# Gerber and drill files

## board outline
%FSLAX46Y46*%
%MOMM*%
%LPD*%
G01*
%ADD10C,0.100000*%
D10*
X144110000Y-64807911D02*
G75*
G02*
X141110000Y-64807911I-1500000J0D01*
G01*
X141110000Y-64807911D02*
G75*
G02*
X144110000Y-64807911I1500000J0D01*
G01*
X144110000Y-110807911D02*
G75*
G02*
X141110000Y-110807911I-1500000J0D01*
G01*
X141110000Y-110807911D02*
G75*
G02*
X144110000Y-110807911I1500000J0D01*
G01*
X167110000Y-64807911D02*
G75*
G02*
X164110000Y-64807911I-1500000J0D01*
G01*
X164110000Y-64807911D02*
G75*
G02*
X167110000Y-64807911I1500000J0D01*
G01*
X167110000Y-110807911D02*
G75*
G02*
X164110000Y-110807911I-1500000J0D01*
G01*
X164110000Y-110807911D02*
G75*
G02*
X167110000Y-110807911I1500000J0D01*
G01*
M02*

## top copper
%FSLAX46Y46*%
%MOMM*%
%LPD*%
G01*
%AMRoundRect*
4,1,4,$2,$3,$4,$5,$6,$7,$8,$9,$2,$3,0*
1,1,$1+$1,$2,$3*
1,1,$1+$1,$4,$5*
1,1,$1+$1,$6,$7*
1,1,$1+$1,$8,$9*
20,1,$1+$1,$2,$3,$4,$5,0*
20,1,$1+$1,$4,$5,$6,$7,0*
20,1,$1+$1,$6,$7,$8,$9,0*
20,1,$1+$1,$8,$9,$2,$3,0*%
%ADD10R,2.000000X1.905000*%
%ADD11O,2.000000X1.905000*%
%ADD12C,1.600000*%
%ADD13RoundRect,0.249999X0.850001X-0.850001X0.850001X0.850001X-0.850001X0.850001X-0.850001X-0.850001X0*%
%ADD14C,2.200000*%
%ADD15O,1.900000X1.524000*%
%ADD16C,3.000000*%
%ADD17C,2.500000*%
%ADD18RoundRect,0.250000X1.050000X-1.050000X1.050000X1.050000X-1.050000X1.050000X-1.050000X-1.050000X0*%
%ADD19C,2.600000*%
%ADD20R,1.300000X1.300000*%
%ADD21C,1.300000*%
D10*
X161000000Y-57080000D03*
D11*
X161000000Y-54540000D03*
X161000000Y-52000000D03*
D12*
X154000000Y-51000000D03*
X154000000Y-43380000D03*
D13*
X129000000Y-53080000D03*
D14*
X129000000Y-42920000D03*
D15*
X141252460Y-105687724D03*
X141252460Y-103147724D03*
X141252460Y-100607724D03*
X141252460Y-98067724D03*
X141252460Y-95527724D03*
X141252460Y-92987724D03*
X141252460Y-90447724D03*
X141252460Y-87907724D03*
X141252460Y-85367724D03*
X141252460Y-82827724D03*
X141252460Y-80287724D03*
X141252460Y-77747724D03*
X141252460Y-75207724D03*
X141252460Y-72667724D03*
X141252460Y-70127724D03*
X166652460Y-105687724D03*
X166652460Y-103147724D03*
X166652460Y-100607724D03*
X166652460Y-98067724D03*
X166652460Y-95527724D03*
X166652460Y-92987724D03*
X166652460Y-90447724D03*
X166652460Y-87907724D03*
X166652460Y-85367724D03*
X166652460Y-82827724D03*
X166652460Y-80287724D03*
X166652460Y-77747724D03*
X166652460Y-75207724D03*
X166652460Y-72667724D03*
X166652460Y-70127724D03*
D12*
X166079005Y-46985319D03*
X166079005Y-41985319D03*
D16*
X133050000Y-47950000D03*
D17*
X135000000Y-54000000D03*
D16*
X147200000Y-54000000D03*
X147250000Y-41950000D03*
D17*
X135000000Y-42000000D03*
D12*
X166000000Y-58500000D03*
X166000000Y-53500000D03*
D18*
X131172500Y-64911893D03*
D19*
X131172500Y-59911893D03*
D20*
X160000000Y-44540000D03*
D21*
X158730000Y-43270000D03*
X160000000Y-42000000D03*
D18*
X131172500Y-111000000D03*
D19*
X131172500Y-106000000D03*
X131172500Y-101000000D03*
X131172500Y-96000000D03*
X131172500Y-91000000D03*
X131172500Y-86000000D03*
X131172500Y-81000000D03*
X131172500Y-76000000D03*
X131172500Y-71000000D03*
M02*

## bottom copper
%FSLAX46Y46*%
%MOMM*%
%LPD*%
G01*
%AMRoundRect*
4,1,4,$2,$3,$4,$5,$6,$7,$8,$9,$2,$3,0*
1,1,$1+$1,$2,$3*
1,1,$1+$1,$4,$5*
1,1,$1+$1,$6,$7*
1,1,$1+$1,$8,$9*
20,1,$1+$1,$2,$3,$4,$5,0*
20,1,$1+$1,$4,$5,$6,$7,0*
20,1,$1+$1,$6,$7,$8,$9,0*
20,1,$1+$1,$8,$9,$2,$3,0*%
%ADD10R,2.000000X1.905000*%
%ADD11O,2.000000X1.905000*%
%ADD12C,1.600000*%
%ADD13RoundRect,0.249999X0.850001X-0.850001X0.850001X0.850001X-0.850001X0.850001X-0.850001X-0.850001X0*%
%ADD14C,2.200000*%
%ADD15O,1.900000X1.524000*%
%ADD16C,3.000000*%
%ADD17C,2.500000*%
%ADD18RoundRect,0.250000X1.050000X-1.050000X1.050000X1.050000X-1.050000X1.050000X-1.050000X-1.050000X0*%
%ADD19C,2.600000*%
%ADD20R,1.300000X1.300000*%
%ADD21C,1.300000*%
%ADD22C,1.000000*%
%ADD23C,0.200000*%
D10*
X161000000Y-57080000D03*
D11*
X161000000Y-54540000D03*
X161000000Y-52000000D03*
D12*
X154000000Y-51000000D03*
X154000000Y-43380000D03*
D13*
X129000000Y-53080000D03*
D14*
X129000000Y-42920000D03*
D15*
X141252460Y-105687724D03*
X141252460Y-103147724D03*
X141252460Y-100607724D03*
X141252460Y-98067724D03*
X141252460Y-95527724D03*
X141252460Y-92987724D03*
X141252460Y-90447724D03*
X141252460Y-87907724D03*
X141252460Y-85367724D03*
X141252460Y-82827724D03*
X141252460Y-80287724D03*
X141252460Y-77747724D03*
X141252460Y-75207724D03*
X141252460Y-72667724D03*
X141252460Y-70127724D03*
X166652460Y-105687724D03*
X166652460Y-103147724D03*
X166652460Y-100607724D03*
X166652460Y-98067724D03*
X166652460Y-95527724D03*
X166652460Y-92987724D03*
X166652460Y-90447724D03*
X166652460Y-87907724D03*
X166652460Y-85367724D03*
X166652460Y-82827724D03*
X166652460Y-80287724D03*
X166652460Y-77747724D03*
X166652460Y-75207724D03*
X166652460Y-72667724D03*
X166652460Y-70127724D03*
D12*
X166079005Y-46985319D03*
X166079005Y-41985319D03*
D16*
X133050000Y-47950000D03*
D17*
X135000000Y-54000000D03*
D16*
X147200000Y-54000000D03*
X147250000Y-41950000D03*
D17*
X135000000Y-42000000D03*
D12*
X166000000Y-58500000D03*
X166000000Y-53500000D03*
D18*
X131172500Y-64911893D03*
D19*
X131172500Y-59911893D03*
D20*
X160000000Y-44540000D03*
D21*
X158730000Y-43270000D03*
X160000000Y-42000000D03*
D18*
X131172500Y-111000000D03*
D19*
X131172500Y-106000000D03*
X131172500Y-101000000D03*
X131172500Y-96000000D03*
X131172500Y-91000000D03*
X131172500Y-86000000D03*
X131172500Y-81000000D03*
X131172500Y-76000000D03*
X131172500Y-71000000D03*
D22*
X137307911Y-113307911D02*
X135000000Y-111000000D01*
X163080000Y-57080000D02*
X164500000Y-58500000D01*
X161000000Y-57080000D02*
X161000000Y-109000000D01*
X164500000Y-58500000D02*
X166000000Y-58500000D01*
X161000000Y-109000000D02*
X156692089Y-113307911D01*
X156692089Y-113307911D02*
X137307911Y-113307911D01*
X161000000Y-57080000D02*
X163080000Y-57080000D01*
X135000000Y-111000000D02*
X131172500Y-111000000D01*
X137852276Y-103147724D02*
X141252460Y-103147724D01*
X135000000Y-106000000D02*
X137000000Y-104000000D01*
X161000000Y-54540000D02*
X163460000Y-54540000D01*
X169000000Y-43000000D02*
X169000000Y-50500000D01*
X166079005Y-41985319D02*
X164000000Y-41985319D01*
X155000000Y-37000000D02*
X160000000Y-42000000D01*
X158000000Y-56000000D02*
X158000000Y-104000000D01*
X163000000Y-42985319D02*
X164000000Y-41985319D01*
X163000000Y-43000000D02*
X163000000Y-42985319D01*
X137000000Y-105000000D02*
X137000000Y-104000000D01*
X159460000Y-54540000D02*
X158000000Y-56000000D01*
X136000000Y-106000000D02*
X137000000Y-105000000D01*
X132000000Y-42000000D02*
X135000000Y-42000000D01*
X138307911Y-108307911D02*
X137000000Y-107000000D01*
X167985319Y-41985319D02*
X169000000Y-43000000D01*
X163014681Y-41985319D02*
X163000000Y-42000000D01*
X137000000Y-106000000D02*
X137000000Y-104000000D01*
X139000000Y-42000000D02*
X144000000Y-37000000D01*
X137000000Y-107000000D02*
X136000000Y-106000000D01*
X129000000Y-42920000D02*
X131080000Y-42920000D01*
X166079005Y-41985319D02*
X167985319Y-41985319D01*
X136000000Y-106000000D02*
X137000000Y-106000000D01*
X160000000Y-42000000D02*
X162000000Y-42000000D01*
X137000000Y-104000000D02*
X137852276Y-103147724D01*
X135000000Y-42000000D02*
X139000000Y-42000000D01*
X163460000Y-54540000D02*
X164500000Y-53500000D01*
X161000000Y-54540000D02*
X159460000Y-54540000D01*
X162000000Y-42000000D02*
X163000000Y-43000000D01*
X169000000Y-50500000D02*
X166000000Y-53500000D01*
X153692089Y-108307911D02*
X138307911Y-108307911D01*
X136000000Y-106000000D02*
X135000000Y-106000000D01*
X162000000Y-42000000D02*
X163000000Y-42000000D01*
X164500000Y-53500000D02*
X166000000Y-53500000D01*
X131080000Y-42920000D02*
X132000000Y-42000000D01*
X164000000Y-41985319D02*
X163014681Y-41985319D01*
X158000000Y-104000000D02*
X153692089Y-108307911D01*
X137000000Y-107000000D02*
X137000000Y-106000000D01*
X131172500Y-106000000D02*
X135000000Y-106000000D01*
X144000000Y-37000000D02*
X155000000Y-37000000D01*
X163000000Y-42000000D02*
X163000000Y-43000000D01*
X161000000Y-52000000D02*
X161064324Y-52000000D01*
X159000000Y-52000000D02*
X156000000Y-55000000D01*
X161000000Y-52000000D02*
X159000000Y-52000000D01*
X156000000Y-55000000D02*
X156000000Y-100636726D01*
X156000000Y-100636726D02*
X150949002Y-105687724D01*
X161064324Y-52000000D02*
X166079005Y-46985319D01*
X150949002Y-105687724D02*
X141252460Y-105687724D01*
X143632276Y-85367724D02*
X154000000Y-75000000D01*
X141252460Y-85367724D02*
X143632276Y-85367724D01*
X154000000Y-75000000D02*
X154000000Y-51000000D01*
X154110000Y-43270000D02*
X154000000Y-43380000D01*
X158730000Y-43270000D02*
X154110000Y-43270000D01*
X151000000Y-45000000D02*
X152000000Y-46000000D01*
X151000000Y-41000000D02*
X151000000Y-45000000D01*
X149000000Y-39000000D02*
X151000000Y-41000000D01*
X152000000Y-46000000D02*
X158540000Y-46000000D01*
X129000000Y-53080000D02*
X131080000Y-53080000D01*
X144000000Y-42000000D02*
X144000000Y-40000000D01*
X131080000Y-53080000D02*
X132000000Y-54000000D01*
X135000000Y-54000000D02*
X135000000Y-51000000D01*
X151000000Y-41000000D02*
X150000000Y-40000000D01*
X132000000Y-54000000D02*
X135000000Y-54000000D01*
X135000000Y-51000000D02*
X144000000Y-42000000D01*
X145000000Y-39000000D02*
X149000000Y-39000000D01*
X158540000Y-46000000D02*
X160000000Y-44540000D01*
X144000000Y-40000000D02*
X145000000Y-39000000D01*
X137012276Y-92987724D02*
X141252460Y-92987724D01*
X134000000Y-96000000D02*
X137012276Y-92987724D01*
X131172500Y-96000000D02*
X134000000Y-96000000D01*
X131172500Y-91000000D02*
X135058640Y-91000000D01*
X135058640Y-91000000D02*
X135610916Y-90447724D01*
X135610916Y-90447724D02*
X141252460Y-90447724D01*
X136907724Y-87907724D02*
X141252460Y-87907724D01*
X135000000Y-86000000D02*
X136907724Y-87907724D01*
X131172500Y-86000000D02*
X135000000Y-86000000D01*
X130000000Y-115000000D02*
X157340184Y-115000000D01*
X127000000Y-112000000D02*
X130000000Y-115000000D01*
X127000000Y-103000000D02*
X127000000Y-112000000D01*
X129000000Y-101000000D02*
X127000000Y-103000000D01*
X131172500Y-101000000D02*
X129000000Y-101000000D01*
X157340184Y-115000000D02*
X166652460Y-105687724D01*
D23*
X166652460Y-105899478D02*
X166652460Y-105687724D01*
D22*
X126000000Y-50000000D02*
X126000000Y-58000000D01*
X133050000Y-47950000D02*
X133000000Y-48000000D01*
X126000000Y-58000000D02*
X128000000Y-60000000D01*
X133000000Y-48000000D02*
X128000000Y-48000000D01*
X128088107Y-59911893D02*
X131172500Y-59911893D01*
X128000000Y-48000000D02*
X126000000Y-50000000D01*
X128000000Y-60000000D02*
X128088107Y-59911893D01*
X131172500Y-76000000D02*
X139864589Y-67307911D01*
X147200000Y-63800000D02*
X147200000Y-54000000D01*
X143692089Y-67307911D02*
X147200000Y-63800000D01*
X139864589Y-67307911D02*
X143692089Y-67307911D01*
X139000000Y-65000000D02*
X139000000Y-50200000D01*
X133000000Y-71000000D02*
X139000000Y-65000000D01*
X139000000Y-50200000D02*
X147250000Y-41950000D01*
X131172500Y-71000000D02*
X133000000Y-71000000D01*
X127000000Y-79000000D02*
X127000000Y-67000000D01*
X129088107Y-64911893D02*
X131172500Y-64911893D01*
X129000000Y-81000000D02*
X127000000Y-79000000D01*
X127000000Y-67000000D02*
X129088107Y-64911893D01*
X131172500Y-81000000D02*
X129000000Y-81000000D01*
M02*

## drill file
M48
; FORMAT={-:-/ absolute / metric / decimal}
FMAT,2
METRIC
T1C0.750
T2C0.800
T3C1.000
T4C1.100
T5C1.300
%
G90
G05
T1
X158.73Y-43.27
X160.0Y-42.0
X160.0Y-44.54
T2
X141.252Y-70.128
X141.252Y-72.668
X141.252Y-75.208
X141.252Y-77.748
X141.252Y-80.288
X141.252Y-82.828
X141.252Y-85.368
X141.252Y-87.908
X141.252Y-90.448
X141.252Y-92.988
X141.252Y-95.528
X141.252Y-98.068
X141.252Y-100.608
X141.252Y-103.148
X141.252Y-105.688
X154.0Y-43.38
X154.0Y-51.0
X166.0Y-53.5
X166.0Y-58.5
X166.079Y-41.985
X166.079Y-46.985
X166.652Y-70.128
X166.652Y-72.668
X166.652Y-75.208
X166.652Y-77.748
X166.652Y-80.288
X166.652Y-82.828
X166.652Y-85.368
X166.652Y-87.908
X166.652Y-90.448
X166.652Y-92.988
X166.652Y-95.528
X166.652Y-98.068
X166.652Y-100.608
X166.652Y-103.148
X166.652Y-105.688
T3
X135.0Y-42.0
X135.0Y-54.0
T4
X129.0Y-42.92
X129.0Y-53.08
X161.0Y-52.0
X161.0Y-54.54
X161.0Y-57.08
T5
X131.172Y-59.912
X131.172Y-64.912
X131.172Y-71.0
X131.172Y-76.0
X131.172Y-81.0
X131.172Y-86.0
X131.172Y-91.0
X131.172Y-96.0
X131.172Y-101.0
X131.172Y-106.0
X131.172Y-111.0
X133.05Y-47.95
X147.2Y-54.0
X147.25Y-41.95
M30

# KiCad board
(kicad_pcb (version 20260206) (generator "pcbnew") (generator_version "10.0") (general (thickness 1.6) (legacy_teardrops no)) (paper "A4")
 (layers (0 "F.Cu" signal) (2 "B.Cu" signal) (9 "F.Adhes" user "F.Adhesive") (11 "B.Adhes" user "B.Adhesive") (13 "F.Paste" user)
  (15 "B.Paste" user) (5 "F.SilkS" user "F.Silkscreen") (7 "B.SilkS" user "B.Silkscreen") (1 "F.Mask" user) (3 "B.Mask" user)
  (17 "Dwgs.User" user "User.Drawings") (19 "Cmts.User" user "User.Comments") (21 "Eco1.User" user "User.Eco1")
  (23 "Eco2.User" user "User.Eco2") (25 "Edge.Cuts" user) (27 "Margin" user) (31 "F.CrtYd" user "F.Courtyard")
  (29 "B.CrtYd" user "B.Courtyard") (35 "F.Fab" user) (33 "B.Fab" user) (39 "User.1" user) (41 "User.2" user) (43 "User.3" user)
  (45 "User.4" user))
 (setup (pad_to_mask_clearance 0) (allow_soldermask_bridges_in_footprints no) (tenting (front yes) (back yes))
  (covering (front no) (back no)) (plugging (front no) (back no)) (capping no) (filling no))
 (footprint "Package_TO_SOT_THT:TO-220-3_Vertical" (layer "F.Cu") (at 161 57.08 90)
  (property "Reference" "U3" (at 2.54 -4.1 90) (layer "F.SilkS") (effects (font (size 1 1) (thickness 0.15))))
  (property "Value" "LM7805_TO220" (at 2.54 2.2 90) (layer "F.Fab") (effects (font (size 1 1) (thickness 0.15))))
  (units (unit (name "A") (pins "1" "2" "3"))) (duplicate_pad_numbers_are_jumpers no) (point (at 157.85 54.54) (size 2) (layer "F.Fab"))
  (pad "1" thru_hole rect (at 0 0 90) (size 1.905 2) (drill 1.1) (layers "*.Cu" "*.Mask") (remove_unused_layers no) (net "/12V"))
  (pad "2" thru_hole oval (at 2.54 0 90) (size 1.905 2) (drill 1.1) (layers "*.Cu" "*.Mask") (remove_unused_layers no) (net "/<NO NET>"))
  (pad "3" thru_hole oval (at 5.08 0 90) (size 1.905 2) (drill 1.1) (layers "*.Cu" "*.Mask") (remove_unused_layers no) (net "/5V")))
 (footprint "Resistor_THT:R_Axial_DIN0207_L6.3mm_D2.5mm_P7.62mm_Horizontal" (layer "F.Cu") (at 154 51 90)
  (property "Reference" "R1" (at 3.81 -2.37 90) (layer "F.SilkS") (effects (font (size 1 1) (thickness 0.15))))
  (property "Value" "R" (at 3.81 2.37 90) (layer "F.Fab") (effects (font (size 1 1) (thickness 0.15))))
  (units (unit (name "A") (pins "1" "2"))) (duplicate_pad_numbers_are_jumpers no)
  (pad "1" thru_hole circle (at 0 0 90) (size 1.6 1.6) (drill 0.8) (layers "*.Cu" "*.Mask") (remove_unused_layers no)
   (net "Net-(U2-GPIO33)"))
  (pad "2" thru_hole circle (at 7.62 0 90) (size 1.6 1.6) (drill 0.8) (layers "*.Cu" "*.Mask") (remove_unused_layers no) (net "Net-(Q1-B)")))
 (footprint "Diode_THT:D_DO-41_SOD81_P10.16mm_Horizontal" (layer "F.Cu") (at 129 53.08 90)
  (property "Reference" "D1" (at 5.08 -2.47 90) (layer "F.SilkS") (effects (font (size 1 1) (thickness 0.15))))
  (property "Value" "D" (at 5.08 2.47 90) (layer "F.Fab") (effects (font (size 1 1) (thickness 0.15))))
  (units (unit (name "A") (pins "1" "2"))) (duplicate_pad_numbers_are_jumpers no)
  (pad "1" thru_hole roundrect (at 0 0 90) (size 2.2 2.2) (drill 1.1) (layers "*.Cu" "*.Mask") (remove_unused_layers no)
   (roundrect_rratio 0.113636) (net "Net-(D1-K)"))
  (pad "2" thru_hole circle (at 10.16 0 90) (size 2.2 2.2) (drill 1.1) (layers "*.Cu" "*.Mask") (remove_unused_layers no) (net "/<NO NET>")))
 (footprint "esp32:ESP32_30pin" (layer "F.Cu") (at 153.18 88.667911)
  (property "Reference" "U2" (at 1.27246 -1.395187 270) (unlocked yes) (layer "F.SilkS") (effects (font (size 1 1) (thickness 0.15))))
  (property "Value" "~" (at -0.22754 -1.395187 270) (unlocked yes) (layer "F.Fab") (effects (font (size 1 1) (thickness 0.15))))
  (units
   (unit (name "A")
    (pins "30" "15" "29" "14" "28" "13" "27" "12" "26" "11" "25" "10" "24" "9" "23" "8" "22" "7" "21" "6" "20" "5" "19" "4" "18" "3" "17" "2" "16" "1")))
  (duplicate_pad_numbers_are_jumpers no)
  (fp_circle (center -10.57 -23.86) (end -10.57 -22.36) (stroke (width 0.1) (type default)) (fill no) (layer "Edge.Cuts"))
  (fp_circle (center -10.57 22.14) (end -10.57 23.64) (stroke (width 0.1) (type default)) (fill no) (layer "Edge.Cuts"))
  (fp_circle (center 12.43 -23.86) (end 12.43 -22.36) (stroke (width 0.1) (type default)) (fill no) (layer "Edge.Cuts"))
  (fp_circle (center 12.43 22.14) (end 12.43 23.64) (stroke (width 0.1) (type default)) (fill no) (layer "Edge.Cuts"))
  (pad "1" thru_hole oval (at -11.92754 17.019813 270) (size 1.524 1.9) (drill 0.8) (layers "*.Cu" "*.Mask") (remove_unused_layers no)
   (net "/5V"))
  (pad "2" thru_hole oval (at -11.92754 14.479813 270) (size 1.524 1.9) (drill 0.8) (layers "*.Cu" "*.Mask") (remove_unused_layers no)
   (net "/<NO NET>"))
  (pad "3" thru_hole oval (at -11.92754 11.939813 270) (size 1.524 1.9) (drill 0.8) (layers "*.Cu" "*.Mask") (remove_unused_layers no)
   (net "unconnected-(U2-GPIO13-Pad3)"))
  (pad "4" thru_hole oval (at -11.92754 9.399813 270) (size 1.524 1.9) (drill 0.8) (layers "*.Cu" "*.Mask") (remove_unused_layers no)
   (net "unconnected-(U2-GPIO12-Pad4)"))
  (pad "5" thru_hole oval (at -11.92754 6.859813 270) (size 1.524 1.9) (drill 0.8) (layers "*.Cu" "*.Mask") (remove_unused_layers no)
   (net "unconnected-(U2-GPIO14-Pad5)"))
  (pad "6" thru_hole oval (at -11.92754 4.319813 270) (size 1.524 1.9) (drill 0.8) (layers "*.Cu" "*.Mask") (remove_unused_layers no)
   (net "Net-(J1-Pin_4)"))
  (pad "7" thru_hole oval (at -11.92754 1.779813 270) (size 1.524 1.9) (drill 0.8) (layers "*.Cu" "*.Mask") (remove_unused_layers no)
   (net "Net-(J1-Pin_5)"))
  (pad "8" thru_hole oval (at -11.92754 -0.760187 270) (size 1.524 1.9) (drill 0.8) (layers "*.Cu" "*.Mask") (remove_unused_layers no)
   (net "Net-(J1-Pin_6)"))
  (pad "9" thru_hole oval (at -11.92754 -3.300187 270) (size 1.524 1.9) (drill 0.8) (layers "*.Cu" "*.Mask") (remove_unused_layers no)
   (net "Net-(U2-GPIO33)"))
  (pad "10" thru_hole oval (at -11.92754 -5.840187 270) (size 1.524 1.9) (drill 0.8) (layers "*.Cu" "*.Mask") (remove_unused_layers no)
   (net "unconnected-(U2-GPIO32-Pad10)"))
  (pad "11" thru_hole oval (at -11.92754 -8.380187 270) (size 1.524 1.9) (drill 0.8) (layers "*.Cu" "*.Mask") (remove_unused_layers no)
   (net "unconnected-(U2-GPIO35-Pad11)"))
  (pad "12" thru_hole oval (at -11.92754 -10.920187 270) (size 1.524 1.9) (drill 0.8) (layers "*.Cu" "*.Mask") (remove_unused_layers no)
   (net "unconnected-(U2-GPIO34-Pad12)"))
  (pad "13" thru_hole oval (at -11.92754 -13.460187 270) (size 1.524 1.9) (drill 0.8) (layers "*.Cu" "*.Mask") (remove_unused_layers no)
   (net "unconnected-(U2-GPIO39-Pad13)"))
  (pad "14" thru_hole oval (at -11.92754 -16.000187 270) (size 1.524 1.9) (drill 0.8) (layers "*.Cu" "*.Mask") (remove_unused_layers no)
   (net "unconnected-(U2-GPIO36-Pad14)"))
  (pad "15" thru_hole oval (at -11.92754 -18.540187 270) (size 1.524 1.9) (drill 0.8) (layers "*.Cu" "*.Mask") (remove_unused_layers no)
   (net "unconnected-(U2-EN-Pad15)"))
  (pad "16" thru_hole oval (at 13.47246 17.019813 270) (size 1.524 1.9) (drill 0.8) (layers "*.Cu" "*.Mask") (remove_unused_layers no)
   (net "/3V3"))
  (pad "17" thru_hole oval (at 13.47246 14.479813 270) (size 1.524 1.9) (drill 0.8) (layers "*.Cu" "*.Mask") (remove_unused_layers no)
   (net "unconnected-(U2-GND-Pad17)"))
  (pad "18" thru_hole oval (at 13.47246 11.939813 270) (size 1.524 1.9) (drill 0.8) (layers "*.Cu" "*.Mask") (remove_unused_layers no)
   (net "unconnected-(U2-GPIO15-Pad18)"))
  (pad "19" thru_hole oval (at 13.47246 9.399813 270) (size 1.524 1.9) (drill 0.8) (layers "*.Cu" "*.Mask") (remove_unused_layers no)
   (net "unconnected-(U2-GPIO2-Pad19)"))
  (pad "20" thru_hole oval (at 13.47246 6.859813 270) (size 1.524 1.9) (drill 0.8) (layers "*.Cu" "*.Mask" "Dwgs.User")
   (remove_unused_layers no) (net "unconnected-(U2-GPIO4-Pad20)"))
  (pad "21" thru_hole oval (at 13.47246 4.319813 270) (size 1.524 1.9) (drill 0.8) (layers "*.Cu" "*.Mask") (remove_unused_layers no)
   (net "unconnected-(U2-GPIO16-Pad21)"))
  (pad "22" thru_hole oval (at 13.47246 1.779813 270) (size 1.524 1.9) (drill 0.8) (layers "*.Cu" "*.Mask") (remove_unused_layers no)
   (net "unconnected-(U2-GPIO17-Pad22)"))
  (pad "23" thru_hole oval (at 13.47246 -0.760187 270) (size 1.524 1.9) (drill 0.8) (layers "*.Cu" "*.Mask") (remove_unused_layers no)
   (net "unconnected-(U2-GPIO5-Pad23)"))
  (pad "24" thru_hole oval (at 13.47246 -3.300187 270) (size 1.524 1.9) (drill 0.8) (layers "*.Cu" "*.Mask") (remove_unused_layers no)
   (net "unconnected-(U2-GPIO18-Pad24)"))
  (pad "25" thru_hole oval (at 13.47246 -5.840187 270) (size 1.524 1.9) (drill 0.8) (layers "*.Cu" "*.Mask") (remove_unused_layers no)
   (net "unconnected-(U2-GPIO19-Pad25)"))
  (pad "26" thru_hole oval (at 13.47246 -8.380187 270) (size 1.524 1.9) (drill 0.8) (layers "*.Cu" "*.Mask") (remove_unused_layers no)
   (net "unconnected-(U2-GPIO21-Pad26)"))
  (pad "27" thru_hole oval (at 13.47246 -10.920187 270) (size 1.524 1.9) (drill 0.8) (layers "*.Cu" "*.Mask") (remove_unused_layers no)
   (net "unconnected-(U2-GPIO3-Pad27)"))
  (pad "28" thru_hole oval (at 13.47246 -13.460187 270) (size 1.524 1.9) (drill 0.8) (layers "*.Cu" "*.Mask") (remove_unused_layers no)
   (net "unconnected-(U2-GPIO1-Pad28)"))
  (pad "29" thru_hole oval (at 13.47246 -16.000187 270) (size 1.524 1.9) (drill 0.8) (layers "*.Cu" "*.Mask") (remove_unused_layers no)
   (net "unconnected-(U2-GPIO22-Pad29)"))
  (pad "30" thru_hole oval (at 13.47246 -18.540187 270) (size 1.524 1.9) (drill 0.8) (layers "*.Cu" "*.Mask") (remove_unused_layers no)
   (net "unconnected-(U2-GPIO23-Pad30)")))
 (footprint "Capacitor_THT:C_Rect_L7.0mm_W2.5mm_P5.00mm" (layer "F.Cu") (at 166.079005 46.985319 90)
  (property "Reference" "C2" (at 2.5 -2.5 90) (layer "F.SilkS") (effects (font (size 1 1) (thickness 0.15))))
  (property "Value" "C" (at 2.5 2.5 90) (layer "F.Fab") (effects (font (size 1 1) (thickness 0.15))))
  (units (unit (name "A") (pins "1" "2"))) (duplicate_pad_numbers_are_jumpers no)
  (pad "1" thru_hole circle (at 0 0 90) (size 1.6 1.6) (drill 0.8) (layers "*.Cu" "*.Mask") (remove_unused_layers no) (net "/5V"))
  (pad "2" thru_hole circle (at 5 0 90) (size 1.6 1.6) (drill 0.8) (layers "*.Cu" "*.Mask") (remove_unused_layers no) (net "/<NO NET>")))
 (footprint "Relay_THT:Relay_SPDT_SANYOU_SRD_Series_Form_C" (layer "F.Cu") (at 133.05 47.95)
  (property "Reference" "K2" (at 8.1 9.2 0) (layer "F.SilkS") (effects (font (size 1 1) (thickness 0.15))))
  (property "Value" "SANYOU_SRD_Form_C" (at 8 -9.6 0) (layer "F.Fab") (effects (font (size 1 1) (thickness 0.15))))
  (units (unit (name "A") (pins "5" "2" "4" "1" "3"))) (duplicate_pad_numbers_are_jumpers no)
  (pad "1" thru_hole circle (at 0 0 90) (size 3 3) (drill 1.3) (layers "*.Cu" "*.Mask") (remove_unused_layers no) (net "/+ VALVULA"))
  (pad "2" thru_hole circle (at 1.95 6.05 90) (size 2.5 2.5) (drill 1) (layers "*.Cu" "*.Mask") (remove_unused_layers no) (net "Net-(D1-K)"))
  (pad "3" thru_hole circle (at 14.15 6.05 90) (size 3 3) (drill 1.3) (layers "*.Cu" "*.Mask") (remove_unused_layers no) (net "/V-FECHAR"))
  (pad "4" thru_hole circle (at 14.2 -6 90) (size 3 3) (drill 1.3) (layers "*.Cu" "*.Mask") (remove_unused_layers no) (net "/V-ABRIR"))
  (pad "5" thru_hole circle (at 1.95 -5.95 90) (size 2.5 2.5) (drill 1) (layers "*.Cu" "*.Mask") (remove_unused_layers no) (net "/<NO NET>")))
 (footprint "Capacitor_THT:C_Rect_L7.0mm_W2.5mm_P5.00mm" (layer "F.Cu") (at 166 58.5 90)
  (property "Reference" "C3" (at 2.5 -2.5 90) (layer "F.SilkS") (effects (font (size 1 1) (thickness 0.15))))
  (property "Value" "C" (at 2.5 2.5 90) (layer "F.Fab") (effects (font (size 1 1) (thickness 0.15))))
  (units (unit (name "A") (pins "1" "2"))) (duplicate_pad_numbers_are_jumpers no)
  (pad "1" thru_hole circle (at 0 0 90) (size 1.6 1.6) (drill 0.8) (layers "*.Cu" "*.Mask") (remove_unused_layers no) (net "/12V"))
  (pad "2" thru_hole circle (at 5 0 90) (size 1.6 1.6) (drill 0.8) (layers "*.Cu" "*.Mask") (remove_unused_layers no) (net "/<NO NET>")))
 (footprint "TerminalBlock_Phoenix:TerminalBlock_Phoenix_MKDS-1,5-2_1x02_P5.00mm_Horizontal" (layer "F.Cu") (at 131.1725 64.911893 90)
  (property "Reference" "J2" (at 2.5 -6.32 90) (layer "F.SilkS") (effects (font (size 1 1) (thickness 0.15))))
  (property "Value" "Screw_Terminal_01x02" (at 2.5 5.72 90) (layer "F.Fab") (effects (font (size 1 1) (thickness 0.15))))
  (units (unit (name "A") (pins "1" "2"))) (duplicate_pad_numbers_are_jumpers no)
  (pad "1" thru_hole roundrect (at 0 0 90) (size 2.6 2.6) (drill 1.3) (layers "*.Cu" "*.Mask") (remove_unused_layers no)
   (roundrect_rratio 0.096154) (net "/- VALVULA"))
  (pad "2" thru_hole circle (at 5 0 90) (size 2.6 2.6) (drill 1.3) (layers "*.Cu" "*.Mask") (remove_unused_layers no) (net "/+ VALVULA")))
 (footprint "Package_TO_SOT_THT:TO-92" (layer "F.Cu") (at 160 44.54 90)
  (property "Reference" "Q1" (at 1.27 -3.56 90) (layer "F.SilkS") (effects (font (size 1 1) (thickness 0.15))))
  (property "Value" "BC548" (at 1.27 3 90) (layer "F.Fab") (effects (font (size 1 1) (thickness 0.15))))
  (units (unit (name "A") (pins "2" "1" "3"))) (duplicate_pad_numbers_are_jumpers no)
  (pad "1" thru_hole rect (at 0 0 90) (size 1.3 1.3) (drill 0.75) (layers "*.Cu" "*.Mask") (remove_unused_layers no) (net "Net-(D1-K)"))
  (pad "2" thru_hole circle (at 1.27 -1.27 90) (size 1.3 1.3) (drill 0.75) (layers "*.Cu" "*.Mask") (remove_unused_layers no)
   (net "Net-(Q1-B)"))
  (pad "3" thru_hole circle (at 2.54 0 90) (size 1.3 1.3) (drill 0.75) (layers "*.Cu" "*.Mask") (remove_unused_layers no) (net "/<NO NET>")))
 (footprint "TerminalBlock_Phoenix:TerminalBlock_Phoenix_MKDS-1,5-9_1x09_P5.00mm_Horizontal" (layer "F.Cu") (at 131.1725 111 90)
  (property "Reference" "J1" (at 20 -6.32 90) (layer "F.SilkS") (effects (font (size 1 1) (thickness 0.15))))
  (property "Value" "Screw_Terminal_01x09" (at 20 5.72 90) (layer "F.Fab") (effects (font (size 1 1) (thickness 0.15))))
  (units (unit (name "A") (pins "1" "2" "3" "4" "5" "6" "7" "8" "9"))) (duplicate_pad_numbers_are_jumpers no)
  (pad "1" thru_hole roundrect (at 0 0 90) (size 2.6 2.6) (drill 1.3) (layers "*.Cu" "*.Mask") (remove_unused_layers no)
   (roundrect_rratio 0.096154) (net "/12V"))
  (pad "2" thru_hole circle (at 5 0 90) (size 2.6 2.6) (drill 1.3) (layers "*.Cu" "*.Mask") (remove_unused_layers no) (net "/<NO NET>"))
  (pad "3" thru_hole circle (at 10 0 90) (size 2.6 2.6) (drill 1.3) (layers "*.Cu" "*.Mask") (remove_unused_layers no) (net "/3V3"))
  (pad "4" thru_hole circle (at 15 0 90) (size 2.6 2.6) (drill 1.3) (layers "*.Cu" "*.Mask") (remove_unused_layers no)
   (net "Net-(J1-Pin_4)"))
  (pad "5" thru_hole circle (at 20 0 90) (size 2.6 2.6) (drill 1.3) (layers "*.Cu" "*.Mask") (remove_unused_layers no)
   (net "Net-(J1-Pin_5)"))
  (pad "6" thru_hole circle (at 25 0 90) (size 2.6 2.6) (drill 1.3) (layers "*.Cu" "*.Mask") (remove_unused_layers no)
   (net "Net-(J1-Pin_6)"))
  (pad "7" thru_hole circle (at 30 0 90) (size 2.6 2.6) (drill 1.3) (layers "*.Cu" "*.Mask") (remove_unused_layers no) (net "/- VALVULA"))
  (pad "8" thru_hole circle (at 35 0 90) (size 2.6 2.6) (drill 1.3) (layers "*.Cu" "*.Mask") (remove_unused_layers no) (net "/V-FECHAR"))
  (pad "9" thru_hole circle (at 40 0 90) (size 2.6 2.6) (drill 1.3) (layers "*.Cu" "*.Mask") (remove_unused_layers no) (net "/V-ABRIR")))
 (segment (start 137.307911 113.307911) (end 135 111) (width 1) (layer "B.Cu") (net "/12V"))
 (segment (start 163.08 57.08) (end 164.5 58.5) (width 1) (layer "B.Cu") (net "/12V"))
 (segment (start 161 57.08) (end 161 109) (width 1) (layer "B.Cu") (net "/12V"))
 (segment (start 164.5 58.5) (end 166 58.5) (width 1) (layer "B.Cu") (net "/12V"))
 (segment (start 161 109) (end 156.692089 113.307911) (width 1) (layer "B.Cu") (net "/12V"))
 (segment (start 156.692089 113.307911) (end 137.307911 113.307911) (width 1) (layer "B.Cu") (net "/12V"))
 (segment (start 161 57.08) (end 163.08 57.08) (width 1) (layer "B.Cu") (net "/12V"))
 (segment (start 135 111) (end 131.1725 111) (width 1) (layer "B.Cu") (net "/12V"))
 (segment (start 137.852276 103.147724) (end 141.25246 103.147724) (width 1) (layer "B.Cu") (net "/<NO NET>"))
 (segment (start 135 106) (end 137 104) (width 1) (layer "B.Cu") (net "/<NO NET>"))
 (segment (start 161 54.54) (end 163.46 54.54) (width 1) (layer "B.Cu") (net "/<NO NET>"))
 (segment (start 169 43) (end 169 50.5) (width 1) (layer "B.Cu") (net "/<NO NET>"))
 (segment (start 166.079005 41.985319) (end 164 41.985319) (width 1) (layer "B.Cu") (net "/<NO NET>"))
 (segment (start 155 37) (end 160 42) (width 1) (layer "B.Cu") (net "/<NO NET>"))
 (segment (start 158 56) (end 158 104) (width 1) (layer "B.Cu") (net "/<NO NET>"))
 (segment (start 163 42.985319) (end 164 41.985319) (width 1) (layer "B.Cu") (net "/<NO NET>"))
 (segment (start 163 43) (end 163 42.985319) (width 1) (layer "B.Cu") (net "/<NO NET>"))
 (segment (start 137 105) (end 137 104) (width 1) (layer "B.Cu") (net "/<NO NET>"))
 (segment (start 159.46 54.54) (end 158 56) (width 1) (layer "B.Cu") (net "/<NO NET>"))
 (segment (start 136 106) (end 137 105) (width 1) (layer "B.Cu") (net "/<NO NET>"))
 (segment (start 132 42) (end 135 42) (width 1) (layer "B.Cu") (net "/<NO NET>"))
 (segment (start 138.307911 108.307911) (end 137 107) (width 1) (layer "B.Cu") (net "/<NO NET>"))
 (segment (start 167.985319 41.985319) (end 169 43) (width 1) (layer "B.Cu") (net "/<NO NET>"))
 (segment (start 163.014681 41.985319) (end 163 42) (width 1) (layer "B.Cu") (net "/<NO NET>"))
 (segment (start 137 106) (end 137 104) (width 1) (layer "B.Cu") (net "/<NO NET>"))
 (segment (start 139 42) (end 144 37) (width 1) (layer "B.Cu") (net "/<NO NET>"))
 (segment (start 137 107) (end 136 106) (width 1) (layer "B.Cu") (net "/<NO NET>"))
 (segment (start 129 42.92) (end 131.08 42.92) (width 1) (layer "B.Cu") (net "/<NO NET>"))
 (segment (start 166.079005 41.985319) (end 167.985319 41.985319) (width 1) (layer "B.Cu") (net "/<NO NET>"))
 (segment (start 136 106) (end 137 106) (width 1) (layer "B.Cu") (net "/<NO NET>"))
 (segment (start 160 42) (end 162 42) (width 1) (layer "B.Cu") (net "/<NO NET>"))
 (segment (start 137 104) (end 137.852276 103.147724) (width 1) (layer "B.Cu") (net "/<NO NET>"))
 (segment (start 135 42) (end 139 42) (width 1) (layer "B.Cu") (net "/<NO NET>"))
 (segment (start 163.46 54.54) (end 164.5 53.5) (width 1) (layer "B.Cu") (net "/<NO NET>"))
 (segment (start 161 54.54) (end 159.46 54.54) (width 1) (layer "B.Cu") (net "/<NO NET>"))
 (segment (start 162 42) (end 163 43) (width 1) (layer "B.Cu") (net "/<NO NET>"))
 (segment (start 169 50.5) (end 166 53.5) (width 1) (layer "B.Cu") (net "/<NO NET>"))
 (segment (start 153.692089 108.307911) (end 138.307911 108.307911) (width 1) (layer "B.Cu") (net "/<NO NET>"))
 (segment (start 136 106) (end 135 106) (width 1) (layer "B.Cu") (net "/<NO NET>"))
 (segment (start 162 42) (end 163 42) (width 1) (layer "B.Cu") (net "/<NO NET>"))
 (segment (start 164.5 53.5) (end 166 53.5) (width 1) (layer "B.Cu") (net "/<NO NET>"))
 (segment (start 131.08 42.92) (end 132 42) (width 1) (layer "B.Cu") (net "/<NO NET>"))
 (segment (start 164 41.985319) (end 163.014681 41.985319) (width 1) (layer "B.Cu") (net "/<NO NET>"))
 (segment (start 158 104) (end 153.692089 108.307911) (width 1) (layer "B.Cu") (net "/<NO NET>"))
 (segment (start 137 107) (end 137 106) (width 1) (layer "B.Cu") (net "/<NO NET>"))
 (segment (start 131.1725 106) (end 135 106) (width 1) (layer "B.Cu") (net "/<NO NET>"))
 (segment (start 144 37) (end 155 37) (width 1) (layer "B.Cu") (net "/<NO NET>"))
 (segment (start 163 42) (end 163 43) (width 1) (layer "B.Cu") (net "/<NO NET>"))
 (segment (start 161 52) (end 161.064324 52) (width 1) (layer "B.Cu") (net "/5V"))
 (segment (start 159 52) (end 156 55) (width 1) (layer "B.Cu") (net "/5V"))
 (segment (start 161 52) (end 159 52) (width 1) (layer "B.Cu") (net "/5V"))
 (segment (start 156 55) (end 156 100.636726) (width 1) (layer "B.Cu") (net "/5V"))
 (segment (start 156 100.636726) (end 150.949002 105.687724) (width 1) (layer "B.Cu") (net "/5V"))
 (segment (start 161.064324 52) (end 166.079005 46.985319) (width 1) (layer "B.Cu") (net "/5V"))
 (segment (start 150.949002 105.687724) (end 141.25246 105.687724) (width 1) (layer "B.Cu") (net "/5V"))
 (segment (start 143.632276 85.367724) (end 154 75) (width 1) (layer "B.Cu") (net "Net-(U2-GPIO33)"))
 (segment (start 141.25246 85.367724) (end 143.632276 85.367724) (width 1) (layer "B.Cu") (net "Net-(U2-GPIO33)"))
 (segment (start 154 75) (end 154 51) (width 1) (layer "B.Cu") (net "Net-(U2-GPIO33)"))
 (segment (start 154.11 43.27) (end 154 43.38) (width 1) (layer "B.Cu") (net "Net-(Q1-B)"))
 (segment (start 158.73 43.27) (end 154.11 43.27) (width 1) (layer "B.Cu") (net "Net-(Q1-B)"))
 (segment (start 151 45) (end 152 46) (width 1) (layer "B.Cu") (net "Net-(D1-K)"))
 (segment (start 151 41) (end 151 45) (width 1) (layer "B.Cu") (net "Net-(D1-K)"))
 (segment (start 149 39) (end 151 41) (width 1) (layer "B.Cu") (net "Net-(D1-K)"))
 (segment (start 152 46) (end 158.54 46) (width 1) (layer "B.Cu") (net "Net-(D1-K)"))
 (segment (start 129 53.08) (end 131.08 53.08) (width 1) (layer "B.Cu") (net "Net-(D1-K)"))
 (segment (start 144 42) (end 144 40) (width 1) (layer "B.Cu") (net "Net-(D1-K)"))
 (segment (start 131.08 53.08) (end 132 54) (width 1) (layer "B.Cu") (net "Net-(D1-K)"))
 (segment (start 135 54) (end 135 51) (width 1) (layer "B.Cu") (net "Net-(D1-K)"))
 (segment (start 151 41) (end 150 40) (width 1) (layer "B.Cu") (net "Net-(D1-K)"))
 (segment (start 132 54) (end 135 54) (width 1) (layer "B.Cu") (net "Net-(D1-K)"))
 (segment (start 135 51) (end 144 42) (width 1) (layer "B.Cu") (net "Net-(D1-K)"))
 (segment (start 145 39) (end 149 39) (width 1) (layer "B.Cu") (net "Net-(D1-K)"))
 (segment (start 158.54 46) (end 160 44.54) (width 1) (layer "B.Cu") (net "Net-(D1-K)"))
 (segment (start 144 40) (end 145 39) (width 1) (layer "B.Cu") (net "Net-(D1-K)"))
 (segment (start 137.012276 92.987724) (end 141.25246 92.987724) (width 1) (layer "B.Cu") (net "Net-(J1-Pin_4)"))
 (segment (start 134 96) (end 137.012276 92.987724) (width 1) (layer "B.Cu") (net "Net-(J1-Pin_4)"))
 (segment (start 131.1725 96) (end 134 96) (width 1) (layer "B.Cu") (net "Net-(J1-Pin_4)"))
 (segment (start 131.1725 91) (end 135.05864 91) (width 1) (layer "B.Cu") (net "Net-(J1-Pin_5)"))
 (segment (start 135.05864 91) (end 135.610916 90.447724) (width 1) (layer "B.Cu") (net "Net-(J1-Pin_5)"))
 (segment (start 135.610916 90.447724) (end 141.25246 90.447724) (width 1) (layer "B.Cu") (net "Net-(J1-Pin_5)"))
 (segment (start 136.907724 87.907724) (end 141.25246 87.907724) (width 1) (layer "B.Cu") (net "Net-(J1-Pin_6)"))
 (segment (start 135 86) (end 136.907724 87.907724) (width 1) (layer "B.Cu") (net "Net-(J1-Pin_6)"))
 (segment (start 131.1725 86) (end 135 86) (width 1) (layer "B.Cu") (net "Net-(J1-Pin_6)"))
 (segment (start 130 115) (end 157.340184 115) (width 1) (layer "B.Cu") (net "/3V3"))
 (segment (start 127 112) (end 130 115) (width 1) (layer "B.Cu") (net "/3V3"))
 (segment (start 127 103) (end 127 112) (width 1) (layer "B.Cu") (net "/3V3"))
 (segment (start 129 101) (end 127 103) (width 1) (layer "B.Cu") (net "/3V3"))
 (segment (start 131.1725 101) (end 129 101) (width 1) (layer "B.Cu") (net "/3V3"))
 (segment (start 157.340184 115) (end 166.65246 105.687724) (width 1) (layer "B.Cu") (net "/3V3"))
 (segment (start 166.65246 105.899478) (end 166.65246 105.687724) (width 0.2) (layer "B.Cu") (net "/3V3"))
 (segment (start 126 50) (end 126 58) (width 1) (layer "B.Cu") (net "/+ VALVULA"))
 (segment (start 133.05 47.95) (end 133 48) (width 1) (layer "B.Cu") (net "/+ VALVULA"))
 (segment (start 126 58) (end 128 60) (width 1) (layer "B.Cu") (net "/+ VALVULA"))
 (segment (start 133 48) (end 128 48) (width 1) (layer "B.Cu") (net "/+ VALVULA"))
 (segment (start 128.088107 59.911893) (end 131.1725 59.911893) (width 1) (layer "B.Cu") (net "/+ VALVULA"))
 (segment (start 128 48) (end 126 50) (width 1) (layer "B.Cu") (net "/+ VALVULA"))
 (segment (start 128 60) (end 128.088107 59.911893) (width 1) (layer "B.Cu") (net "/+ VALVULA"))
 (segment (start 131.1725 76) (end 139.864589 67.307911) (width 1) (layer "B.Cu") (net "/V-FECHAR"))
 (segment (start 147.2 63.8) (end 147.2 54) (width 1) (layer "B.Cu") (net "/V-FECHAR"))
 (segment (start 143.692089 67.307911) (end 147.2 63.8) (width 1) (layer "B.Cu") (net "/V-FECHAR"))
 (segment (start 139.864589 67.307911) (end 143.692089 67.307911) (width 1) (layer "B.Cu") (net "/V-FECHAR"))
 (segment (start 139 65) (end 139 50.2) (width 1) (layer "B.Cu") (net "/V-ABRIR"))
 (segment (start 133 71) (end 139 65) (width 1) (layer "B.Cu") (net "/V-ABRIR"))
 (segment (start 139 50.2) (end 147.25 41.95) (width 1) (layer "B.Cu") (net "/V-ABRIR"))
 (segment (start 131.1725 71) (end 133 71) (width 1) (layer "B.Cu") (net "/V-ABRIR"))
 (segment (start 127 79) (end 127 67) (width 1) (layer "B.Cu") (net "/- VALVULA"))
 (segment (start 129.088107 64.911893) (end 131.1725 64.911893) (width 1) (layer "B.Cu") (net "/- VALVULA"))
 (segment (start 129 81) (end 127 79) (width 1) (layer "B.Cu") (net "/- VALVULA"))
 (segment (start 127 67) (end 129.088107 64.911893) (width 1) (layer "B.Cu") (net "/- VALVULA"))
 (segment (start 131.1725 81) (end 129 81) (width 1) (layer "B.Cu") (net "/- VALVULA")))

